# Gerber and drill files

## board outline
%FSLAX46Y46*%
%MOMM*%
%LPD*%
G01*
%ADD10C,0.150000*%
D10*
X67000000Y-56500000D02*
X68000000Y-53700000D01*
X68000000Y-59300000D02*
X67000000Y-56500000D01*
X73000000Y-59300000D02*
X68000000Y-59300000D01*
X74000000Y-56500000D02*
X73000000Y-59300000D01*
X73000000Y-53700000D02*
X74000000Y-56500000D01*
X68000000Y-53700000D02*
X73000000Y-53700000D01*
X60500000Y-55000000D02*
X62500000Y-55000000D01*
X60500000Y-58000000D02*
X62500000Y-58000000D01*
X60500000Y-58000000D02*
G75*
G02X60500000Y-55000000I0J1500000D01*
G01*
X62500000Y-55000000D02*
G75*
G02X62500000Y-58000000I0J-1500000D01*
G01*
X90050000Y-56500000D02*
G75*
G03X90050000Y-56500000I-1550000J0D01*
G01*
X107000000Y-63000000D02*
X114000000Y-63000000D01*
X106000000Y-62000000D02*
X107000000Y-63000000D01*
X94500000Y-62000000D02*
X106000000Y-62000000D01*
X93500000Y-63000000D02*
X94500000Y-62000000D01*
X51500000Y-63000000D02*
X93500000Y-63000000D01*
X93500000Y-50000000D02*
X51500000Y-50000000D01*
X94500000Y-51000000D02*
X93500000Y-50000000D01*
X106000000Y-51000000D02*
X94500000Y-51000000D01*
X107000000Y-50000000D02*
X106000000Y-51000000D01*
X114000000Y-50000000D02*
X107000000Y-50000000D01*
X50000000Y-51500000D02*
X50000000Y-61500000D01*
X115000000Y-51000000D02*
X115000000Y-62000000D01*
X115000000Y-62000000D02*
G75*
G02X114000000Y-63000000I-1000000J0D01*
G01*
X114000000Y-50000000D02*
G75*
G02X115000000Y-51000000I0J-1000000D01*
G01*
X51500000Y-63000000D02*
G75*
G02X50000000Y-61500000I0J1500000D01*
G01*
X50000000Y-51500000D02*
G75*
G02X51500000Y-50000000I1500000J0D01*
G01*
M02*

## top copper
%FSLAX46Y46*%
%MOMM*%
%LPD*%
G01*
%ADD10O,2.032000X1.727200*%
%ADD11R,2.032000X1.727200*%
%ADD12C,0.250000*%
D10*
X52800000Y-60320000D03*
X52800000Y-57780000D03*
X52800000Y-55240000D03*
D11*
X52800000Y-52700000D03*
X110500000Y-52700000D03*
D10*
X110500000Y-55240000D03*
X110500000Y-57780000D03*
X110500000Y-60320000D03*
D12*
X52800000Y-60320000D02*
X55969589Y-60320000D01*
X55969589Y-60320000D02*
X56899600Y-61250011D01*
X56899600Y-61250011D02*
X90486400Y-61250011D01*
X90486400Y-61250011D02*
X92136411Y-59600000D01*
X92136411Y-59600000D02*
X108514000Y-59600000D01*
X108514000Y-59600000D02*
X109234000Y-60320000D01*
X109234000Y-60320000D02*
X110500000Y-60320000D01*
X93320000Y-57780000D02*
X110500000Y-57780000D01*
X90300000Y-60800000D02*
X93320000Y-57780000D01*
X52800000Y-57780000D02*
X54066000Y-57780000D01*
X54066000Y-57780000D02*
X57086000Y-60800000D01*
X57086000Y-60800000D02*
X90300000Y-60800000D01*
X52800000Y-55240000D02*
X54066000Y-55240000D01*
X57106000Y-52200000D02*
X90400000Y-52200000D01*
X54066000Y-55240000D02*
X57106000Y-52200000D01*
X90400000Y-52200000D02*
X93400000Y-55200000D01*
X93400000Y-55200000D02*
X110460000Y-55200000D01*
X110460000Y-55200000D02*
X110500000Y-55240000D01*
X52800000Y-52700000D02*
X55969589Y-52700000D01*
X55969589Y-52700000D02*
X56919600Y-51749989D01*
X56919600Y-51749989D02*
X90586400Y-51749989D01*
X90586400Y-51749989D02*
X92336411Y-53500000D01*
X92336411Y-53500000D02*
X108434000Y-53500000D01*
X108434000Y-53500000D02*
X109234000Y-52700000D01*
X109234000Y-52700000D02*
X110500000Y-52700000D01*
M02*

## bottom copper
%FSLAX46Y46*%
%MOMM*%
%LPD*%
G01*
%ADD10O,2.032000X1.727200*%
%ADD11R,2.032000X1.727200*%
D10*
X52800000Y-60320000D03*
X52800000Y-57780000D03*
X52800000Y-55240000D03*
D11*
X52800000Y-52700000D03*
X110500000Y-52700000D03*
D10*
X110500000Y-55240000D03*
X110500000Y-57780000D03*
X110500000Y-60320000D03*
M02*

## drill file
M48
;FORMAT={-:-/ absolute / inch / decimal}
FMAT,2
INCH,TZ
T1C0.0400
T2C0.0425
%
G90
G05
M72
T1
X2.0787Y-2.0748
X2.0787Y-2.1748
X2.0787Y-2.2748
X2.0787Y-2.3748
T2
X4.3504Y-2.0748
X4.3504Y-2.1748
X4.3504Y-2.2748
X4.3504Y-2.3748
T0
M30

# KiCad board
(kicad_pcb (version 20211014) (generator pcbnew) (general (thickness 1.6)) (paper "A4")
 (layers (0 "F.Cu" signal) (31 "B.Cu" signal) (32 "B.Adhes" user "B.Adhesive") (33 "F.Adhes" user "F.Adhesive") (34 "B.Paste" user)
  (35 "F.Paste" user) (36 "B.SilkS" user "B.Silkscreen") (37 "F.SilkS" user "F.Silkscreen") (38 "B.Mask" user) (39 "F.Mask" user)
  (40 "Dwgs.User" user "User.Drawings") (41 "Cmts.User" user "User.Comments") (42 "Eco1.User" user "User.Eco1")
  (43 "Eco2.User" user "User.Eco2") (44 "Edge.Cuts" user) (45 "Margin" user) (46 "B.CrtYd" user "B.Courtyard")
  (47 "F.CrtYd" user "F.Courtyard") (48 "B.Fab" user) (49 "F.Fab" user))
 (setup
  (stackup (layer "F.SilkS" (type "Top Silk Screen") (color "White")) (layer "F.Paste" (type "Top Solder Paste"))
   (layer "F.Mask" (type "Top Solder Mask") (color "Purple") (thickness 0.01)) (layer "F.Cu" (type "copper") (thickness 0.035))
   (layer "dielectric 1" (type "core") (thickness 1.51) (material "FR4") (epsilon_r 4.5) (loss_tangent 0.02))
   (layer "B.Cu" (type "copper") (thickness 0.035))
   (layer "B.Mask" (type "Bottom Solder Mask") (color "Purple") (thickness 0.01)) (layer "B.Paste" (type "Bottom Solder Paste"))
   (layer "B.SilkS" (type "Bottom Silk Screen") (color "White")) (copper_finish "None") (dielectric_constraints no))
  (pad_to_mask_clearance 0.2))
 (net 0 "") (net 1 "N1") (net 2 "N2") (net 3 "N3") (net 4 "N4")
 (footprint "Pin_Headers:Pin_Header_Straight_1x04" (layer "F.Cu") (at 52.8 52.7)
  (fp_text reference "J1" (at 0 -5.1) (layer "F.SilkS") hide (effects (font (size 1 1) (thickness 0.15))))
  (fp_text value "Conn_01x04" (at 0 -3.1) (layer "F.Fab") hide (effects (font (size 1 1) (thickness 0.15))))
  (pad "1" thru_hole rect locked (at 0 0) (size 2.032 1.7272) (drill 1.016) (layers *.Cu *.Mask) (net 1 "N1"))
  (pad "2" thru_hole oval locked (at 0 2.54) (size 2.032 1.7272) (drill 1.016) (layers *.Cu *.Mask) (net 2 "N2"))
  (pad "3" thru_hole oval locked (at 0 5.08) (size 2.032 1.7272) (drill 1.016) (layers *.Cu *.Mask) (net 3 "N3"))
  (pad "4" thru_hole oval locked (at 0 7.62) (size 2.032 1.7272) (drill 1.016) (layers *.Cu *.Mask) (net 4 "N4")))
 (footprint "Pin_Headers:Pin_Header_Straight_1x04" (layer "F.Cu") (at 110.5 52.7)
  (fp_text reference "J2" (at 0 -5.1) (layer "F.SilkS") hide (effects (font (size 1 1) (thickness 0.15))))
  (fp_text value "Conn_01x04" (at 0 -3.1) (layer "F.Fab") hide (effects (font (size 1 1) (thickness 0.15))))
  (pad "1" thru_hole rect locked (at 0 0) (size 2.032 1.7272) (drill 1.08) (layers *.Cu *.Mask) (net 1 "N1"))
  (pad "2" thru_hole oval locked (at 0 2.54) (size 2.032 1.7272) (drill 1.08) (layers *.Cu *.Mask) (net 2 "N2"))
  (pad "3" thru_hole oval locked (at 0 5.08) (size 2.032 1.7272) (drill 1.08) (layers *.Cu *.Mask) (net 3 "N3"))
  (pad "4" thru_hole oval locked (at 0 7.62) (size 2.032 1.7272) (drill 1.08) (layers *.Cu *.Mask) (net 4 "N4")))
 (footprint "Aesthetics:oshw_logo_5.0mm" (layer "F.Cu") (at 100.5 56.5 -90)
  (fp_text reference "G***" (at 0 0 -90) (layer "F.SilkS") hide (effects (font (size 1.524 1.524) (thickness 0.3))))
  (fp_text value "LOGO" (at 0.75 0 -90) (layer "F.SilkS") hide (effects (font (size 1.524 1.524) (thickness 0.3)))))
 (gr_arc (start 60.5 58) (mid 59 56.5) (end 60.5 55) (layer "Edge.Cuts") (width 0.15))
 (gr_line (start 115 51) (end 115 62) (layer "Edge.Cuts") (width 0.15))
 (gr_line (start 68 53.7) (end 73 53.7) (layer "Edge.Cuts") (width 0.15))
 (gr_arc (start 62.5 55) (mid 64 56.5) (end 62.5 58) (layer "Edge.Cuts") (width 0.15))
 (gr_line (start 73 53.7) (end 74 56.5) (layer "Edge.Cuts") (width 0.15))
 (gr_line (start 60.5 58) (end 62.5 58) (layer "Edge.Cuts") (width 0.15))
 (gr_line (start 107 50) (end 106 51) (layer "Edge.Cuts") (width 0.15))
 (gr_circle (center 88.5 56.5) (end 90.05 56.5) (layer "Edge.Cuts") (width 0.15) (fill none))
 (gr_line (start 68 59.3) (end 67 56.5) (layer "Edge.Cuts") (width 0.15))
 (gr_line (start 94.5 62) (end 106 62) (layer "Edge.Cuts") (width 0.15))
 (gr_line (start 94.5 51) (end 93.5 50) (layer "Edge.Cuts") (width 0.15))
 (gr_line (start 51.5 63) (end 93.5 63) (layer "Edge.Cuts") (width 0.15))
 (gr_line (start 67 56.5) (end 68 53.7) (layer "Edge.Cuts") (width 0.15))
 (gr_line (start 93.5 50) (end 51.5 50) (layer "Edge.Cuts") (width 0.15))
 (gr_line (start 60.5 55) (end 62.5 55) (layer "Edge.Cuts") (width 0.15))
 (gr_arc (start 115 62) (mid 114.707107 62.707107) (end 114 63) (layer "Edge.Cuts") (width 0.15))
 (gr_line (start 74 56.5) (end 73 59.3) (layer "Edge.Cuts") (width 0.15))
 (gr_line (start 106 51) (end 94.5 51) (layer "Edge.Cuts") (width 0.15))
 (gr_arc (start 51.5 63) (mid 50.43934 62.56066) (end 50 61.5) (layer "Edge.Cuts") (width 0.15))
 (gr_line (start 107 63) (end 114 63) (layer "Edge.Cuts") (width 0.15))
 (gr_arc (start 50 51.5) (mid 50.43934 50.43934) (end 51.5 50) (layer "Edge.Cuts") (width 0.15))
 (gr_line (start 50 51.5) (end 50 61.5) (layer "Edge.Cuts") (width 0.15))
 (gr_arc (start 114 50) (mid 114.707107 50.292893) (end 115 51) (layer "Edge.Cuts") (width 0.15))
 (gr_line (start 73 59.3) (end 68 59.3) (layer "Edge.Cuts") (width 0.15))
 (gr_line (start 114 50) (end 107 50) (layer "Edge.Cuts") (width 0.15))
 (gr_line (start 106 62) (end 107 63) (layer "Edge.Cuts") (width 0.15))
 (gr_line (start 93.5 63) (end 94.5 62) (layer "Edge.Cuts") (width 0.15))
 (segment (start 90.4864 61.250011) (end 92.136411 59.6) (width 0.25) (layer "F.Cu") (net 4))
 (segment (start 55.969589 60.32) (end 56.8996 61.250011) (width 0.25) (layer "F.Cu") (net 4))
 (segment (start 109.234 60.32) (end 110.5 60.32) (width 0.25) (layer "F.Cu") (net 4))
 (segment (start 92.136411 59.6) (end 108.514 59.6) (width 0.25) (layer "F.Cu") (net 4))
 (segment (start 108.514 59.6) (end 109.234 60.32) (width 0.25) (layer "F.Cu") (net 4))
 (segment (start 52.8 60.32) (end 55.969589 60.32) (width 0.25) (layer "F.Cu") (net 4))
 (segment (start 56.8996 61.250011) (end 90.4864 61.250011) (width 0.25) (layer "F.Cu") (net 4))
 (segment (start 57.086 60.8) (end 90.3 60.8) (width 0.25) (layer "F.Cu") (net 3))
 (segment (start 93.32 57.78) (end 110.5 57.78) (width 0.25) (layer "F.Cu") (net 3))
 (segment (start 52.8 57.78) (end 54.066 57.78) (width 0.25) (layer "F.Cu") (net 3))
 (segment (start 54.066 57.78) (end 57.086 60.8) (width 0.25) (layer "F.Cu") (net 3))
 (segment (start 90.3 60.8) (end 93.32 57.78) (width 0.25) (layer "F.Cu") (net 3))
 (segment (start 57.106 52.2) (end 90.4 52.2) (width 0.25) (layer "F.Cu") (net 2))
 (segment (start 90.4 52.2) (end 93.4 55.2) (width 0.25) (layer "F.Cu") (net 2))
 (segment (start 52.8 55.24) (end 54.066 55.24) (width 0.25) (layer "F.Cu") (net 2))
 (segment (start 54.066 55.24) (end 57.106 52.2) (width 0.25) (layer "F.Cu") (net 2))
 (segment (start 110.46 55.2) (end 110.5 55.24) (width 0.25) (layer "F.Cu") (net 2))
 (segment (start 93.4 55.2) (end 110.46 55.2) (width 0.25) (layer "F.Cu") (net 2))
 (segment (start 92.336411 53.5) (end 108.434 53.5) (width 0.25) (layer "F.Cu") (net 1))
 (segment (start 56.9196 51.749989) (end 90.5864 51.749989) (width 0.25) (layer "F.Cu") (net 1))
 (segment (start 90.5864 51.749989) (end 92.336411 53.5) (width 0.25) (layer "F.Cu") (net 1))
 (segment (start 52.8 52.7) (end 55.969589 52.7) (width 0.25) (layer "F.Cu") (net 1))
 (segment (start 109.234 52.7) (end 110.5 52.7) (width 0.25) (layer "F.Cu") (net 1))
 (segment (start 55.969589 52.7) (end 56.9196 51.749989) (width 0.25) (layer "F.Cu") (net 1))
 (segment (start 108.434 53.5) (end 109.234 52.7) (width 0.25) (layer "F.Cu") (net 1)))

